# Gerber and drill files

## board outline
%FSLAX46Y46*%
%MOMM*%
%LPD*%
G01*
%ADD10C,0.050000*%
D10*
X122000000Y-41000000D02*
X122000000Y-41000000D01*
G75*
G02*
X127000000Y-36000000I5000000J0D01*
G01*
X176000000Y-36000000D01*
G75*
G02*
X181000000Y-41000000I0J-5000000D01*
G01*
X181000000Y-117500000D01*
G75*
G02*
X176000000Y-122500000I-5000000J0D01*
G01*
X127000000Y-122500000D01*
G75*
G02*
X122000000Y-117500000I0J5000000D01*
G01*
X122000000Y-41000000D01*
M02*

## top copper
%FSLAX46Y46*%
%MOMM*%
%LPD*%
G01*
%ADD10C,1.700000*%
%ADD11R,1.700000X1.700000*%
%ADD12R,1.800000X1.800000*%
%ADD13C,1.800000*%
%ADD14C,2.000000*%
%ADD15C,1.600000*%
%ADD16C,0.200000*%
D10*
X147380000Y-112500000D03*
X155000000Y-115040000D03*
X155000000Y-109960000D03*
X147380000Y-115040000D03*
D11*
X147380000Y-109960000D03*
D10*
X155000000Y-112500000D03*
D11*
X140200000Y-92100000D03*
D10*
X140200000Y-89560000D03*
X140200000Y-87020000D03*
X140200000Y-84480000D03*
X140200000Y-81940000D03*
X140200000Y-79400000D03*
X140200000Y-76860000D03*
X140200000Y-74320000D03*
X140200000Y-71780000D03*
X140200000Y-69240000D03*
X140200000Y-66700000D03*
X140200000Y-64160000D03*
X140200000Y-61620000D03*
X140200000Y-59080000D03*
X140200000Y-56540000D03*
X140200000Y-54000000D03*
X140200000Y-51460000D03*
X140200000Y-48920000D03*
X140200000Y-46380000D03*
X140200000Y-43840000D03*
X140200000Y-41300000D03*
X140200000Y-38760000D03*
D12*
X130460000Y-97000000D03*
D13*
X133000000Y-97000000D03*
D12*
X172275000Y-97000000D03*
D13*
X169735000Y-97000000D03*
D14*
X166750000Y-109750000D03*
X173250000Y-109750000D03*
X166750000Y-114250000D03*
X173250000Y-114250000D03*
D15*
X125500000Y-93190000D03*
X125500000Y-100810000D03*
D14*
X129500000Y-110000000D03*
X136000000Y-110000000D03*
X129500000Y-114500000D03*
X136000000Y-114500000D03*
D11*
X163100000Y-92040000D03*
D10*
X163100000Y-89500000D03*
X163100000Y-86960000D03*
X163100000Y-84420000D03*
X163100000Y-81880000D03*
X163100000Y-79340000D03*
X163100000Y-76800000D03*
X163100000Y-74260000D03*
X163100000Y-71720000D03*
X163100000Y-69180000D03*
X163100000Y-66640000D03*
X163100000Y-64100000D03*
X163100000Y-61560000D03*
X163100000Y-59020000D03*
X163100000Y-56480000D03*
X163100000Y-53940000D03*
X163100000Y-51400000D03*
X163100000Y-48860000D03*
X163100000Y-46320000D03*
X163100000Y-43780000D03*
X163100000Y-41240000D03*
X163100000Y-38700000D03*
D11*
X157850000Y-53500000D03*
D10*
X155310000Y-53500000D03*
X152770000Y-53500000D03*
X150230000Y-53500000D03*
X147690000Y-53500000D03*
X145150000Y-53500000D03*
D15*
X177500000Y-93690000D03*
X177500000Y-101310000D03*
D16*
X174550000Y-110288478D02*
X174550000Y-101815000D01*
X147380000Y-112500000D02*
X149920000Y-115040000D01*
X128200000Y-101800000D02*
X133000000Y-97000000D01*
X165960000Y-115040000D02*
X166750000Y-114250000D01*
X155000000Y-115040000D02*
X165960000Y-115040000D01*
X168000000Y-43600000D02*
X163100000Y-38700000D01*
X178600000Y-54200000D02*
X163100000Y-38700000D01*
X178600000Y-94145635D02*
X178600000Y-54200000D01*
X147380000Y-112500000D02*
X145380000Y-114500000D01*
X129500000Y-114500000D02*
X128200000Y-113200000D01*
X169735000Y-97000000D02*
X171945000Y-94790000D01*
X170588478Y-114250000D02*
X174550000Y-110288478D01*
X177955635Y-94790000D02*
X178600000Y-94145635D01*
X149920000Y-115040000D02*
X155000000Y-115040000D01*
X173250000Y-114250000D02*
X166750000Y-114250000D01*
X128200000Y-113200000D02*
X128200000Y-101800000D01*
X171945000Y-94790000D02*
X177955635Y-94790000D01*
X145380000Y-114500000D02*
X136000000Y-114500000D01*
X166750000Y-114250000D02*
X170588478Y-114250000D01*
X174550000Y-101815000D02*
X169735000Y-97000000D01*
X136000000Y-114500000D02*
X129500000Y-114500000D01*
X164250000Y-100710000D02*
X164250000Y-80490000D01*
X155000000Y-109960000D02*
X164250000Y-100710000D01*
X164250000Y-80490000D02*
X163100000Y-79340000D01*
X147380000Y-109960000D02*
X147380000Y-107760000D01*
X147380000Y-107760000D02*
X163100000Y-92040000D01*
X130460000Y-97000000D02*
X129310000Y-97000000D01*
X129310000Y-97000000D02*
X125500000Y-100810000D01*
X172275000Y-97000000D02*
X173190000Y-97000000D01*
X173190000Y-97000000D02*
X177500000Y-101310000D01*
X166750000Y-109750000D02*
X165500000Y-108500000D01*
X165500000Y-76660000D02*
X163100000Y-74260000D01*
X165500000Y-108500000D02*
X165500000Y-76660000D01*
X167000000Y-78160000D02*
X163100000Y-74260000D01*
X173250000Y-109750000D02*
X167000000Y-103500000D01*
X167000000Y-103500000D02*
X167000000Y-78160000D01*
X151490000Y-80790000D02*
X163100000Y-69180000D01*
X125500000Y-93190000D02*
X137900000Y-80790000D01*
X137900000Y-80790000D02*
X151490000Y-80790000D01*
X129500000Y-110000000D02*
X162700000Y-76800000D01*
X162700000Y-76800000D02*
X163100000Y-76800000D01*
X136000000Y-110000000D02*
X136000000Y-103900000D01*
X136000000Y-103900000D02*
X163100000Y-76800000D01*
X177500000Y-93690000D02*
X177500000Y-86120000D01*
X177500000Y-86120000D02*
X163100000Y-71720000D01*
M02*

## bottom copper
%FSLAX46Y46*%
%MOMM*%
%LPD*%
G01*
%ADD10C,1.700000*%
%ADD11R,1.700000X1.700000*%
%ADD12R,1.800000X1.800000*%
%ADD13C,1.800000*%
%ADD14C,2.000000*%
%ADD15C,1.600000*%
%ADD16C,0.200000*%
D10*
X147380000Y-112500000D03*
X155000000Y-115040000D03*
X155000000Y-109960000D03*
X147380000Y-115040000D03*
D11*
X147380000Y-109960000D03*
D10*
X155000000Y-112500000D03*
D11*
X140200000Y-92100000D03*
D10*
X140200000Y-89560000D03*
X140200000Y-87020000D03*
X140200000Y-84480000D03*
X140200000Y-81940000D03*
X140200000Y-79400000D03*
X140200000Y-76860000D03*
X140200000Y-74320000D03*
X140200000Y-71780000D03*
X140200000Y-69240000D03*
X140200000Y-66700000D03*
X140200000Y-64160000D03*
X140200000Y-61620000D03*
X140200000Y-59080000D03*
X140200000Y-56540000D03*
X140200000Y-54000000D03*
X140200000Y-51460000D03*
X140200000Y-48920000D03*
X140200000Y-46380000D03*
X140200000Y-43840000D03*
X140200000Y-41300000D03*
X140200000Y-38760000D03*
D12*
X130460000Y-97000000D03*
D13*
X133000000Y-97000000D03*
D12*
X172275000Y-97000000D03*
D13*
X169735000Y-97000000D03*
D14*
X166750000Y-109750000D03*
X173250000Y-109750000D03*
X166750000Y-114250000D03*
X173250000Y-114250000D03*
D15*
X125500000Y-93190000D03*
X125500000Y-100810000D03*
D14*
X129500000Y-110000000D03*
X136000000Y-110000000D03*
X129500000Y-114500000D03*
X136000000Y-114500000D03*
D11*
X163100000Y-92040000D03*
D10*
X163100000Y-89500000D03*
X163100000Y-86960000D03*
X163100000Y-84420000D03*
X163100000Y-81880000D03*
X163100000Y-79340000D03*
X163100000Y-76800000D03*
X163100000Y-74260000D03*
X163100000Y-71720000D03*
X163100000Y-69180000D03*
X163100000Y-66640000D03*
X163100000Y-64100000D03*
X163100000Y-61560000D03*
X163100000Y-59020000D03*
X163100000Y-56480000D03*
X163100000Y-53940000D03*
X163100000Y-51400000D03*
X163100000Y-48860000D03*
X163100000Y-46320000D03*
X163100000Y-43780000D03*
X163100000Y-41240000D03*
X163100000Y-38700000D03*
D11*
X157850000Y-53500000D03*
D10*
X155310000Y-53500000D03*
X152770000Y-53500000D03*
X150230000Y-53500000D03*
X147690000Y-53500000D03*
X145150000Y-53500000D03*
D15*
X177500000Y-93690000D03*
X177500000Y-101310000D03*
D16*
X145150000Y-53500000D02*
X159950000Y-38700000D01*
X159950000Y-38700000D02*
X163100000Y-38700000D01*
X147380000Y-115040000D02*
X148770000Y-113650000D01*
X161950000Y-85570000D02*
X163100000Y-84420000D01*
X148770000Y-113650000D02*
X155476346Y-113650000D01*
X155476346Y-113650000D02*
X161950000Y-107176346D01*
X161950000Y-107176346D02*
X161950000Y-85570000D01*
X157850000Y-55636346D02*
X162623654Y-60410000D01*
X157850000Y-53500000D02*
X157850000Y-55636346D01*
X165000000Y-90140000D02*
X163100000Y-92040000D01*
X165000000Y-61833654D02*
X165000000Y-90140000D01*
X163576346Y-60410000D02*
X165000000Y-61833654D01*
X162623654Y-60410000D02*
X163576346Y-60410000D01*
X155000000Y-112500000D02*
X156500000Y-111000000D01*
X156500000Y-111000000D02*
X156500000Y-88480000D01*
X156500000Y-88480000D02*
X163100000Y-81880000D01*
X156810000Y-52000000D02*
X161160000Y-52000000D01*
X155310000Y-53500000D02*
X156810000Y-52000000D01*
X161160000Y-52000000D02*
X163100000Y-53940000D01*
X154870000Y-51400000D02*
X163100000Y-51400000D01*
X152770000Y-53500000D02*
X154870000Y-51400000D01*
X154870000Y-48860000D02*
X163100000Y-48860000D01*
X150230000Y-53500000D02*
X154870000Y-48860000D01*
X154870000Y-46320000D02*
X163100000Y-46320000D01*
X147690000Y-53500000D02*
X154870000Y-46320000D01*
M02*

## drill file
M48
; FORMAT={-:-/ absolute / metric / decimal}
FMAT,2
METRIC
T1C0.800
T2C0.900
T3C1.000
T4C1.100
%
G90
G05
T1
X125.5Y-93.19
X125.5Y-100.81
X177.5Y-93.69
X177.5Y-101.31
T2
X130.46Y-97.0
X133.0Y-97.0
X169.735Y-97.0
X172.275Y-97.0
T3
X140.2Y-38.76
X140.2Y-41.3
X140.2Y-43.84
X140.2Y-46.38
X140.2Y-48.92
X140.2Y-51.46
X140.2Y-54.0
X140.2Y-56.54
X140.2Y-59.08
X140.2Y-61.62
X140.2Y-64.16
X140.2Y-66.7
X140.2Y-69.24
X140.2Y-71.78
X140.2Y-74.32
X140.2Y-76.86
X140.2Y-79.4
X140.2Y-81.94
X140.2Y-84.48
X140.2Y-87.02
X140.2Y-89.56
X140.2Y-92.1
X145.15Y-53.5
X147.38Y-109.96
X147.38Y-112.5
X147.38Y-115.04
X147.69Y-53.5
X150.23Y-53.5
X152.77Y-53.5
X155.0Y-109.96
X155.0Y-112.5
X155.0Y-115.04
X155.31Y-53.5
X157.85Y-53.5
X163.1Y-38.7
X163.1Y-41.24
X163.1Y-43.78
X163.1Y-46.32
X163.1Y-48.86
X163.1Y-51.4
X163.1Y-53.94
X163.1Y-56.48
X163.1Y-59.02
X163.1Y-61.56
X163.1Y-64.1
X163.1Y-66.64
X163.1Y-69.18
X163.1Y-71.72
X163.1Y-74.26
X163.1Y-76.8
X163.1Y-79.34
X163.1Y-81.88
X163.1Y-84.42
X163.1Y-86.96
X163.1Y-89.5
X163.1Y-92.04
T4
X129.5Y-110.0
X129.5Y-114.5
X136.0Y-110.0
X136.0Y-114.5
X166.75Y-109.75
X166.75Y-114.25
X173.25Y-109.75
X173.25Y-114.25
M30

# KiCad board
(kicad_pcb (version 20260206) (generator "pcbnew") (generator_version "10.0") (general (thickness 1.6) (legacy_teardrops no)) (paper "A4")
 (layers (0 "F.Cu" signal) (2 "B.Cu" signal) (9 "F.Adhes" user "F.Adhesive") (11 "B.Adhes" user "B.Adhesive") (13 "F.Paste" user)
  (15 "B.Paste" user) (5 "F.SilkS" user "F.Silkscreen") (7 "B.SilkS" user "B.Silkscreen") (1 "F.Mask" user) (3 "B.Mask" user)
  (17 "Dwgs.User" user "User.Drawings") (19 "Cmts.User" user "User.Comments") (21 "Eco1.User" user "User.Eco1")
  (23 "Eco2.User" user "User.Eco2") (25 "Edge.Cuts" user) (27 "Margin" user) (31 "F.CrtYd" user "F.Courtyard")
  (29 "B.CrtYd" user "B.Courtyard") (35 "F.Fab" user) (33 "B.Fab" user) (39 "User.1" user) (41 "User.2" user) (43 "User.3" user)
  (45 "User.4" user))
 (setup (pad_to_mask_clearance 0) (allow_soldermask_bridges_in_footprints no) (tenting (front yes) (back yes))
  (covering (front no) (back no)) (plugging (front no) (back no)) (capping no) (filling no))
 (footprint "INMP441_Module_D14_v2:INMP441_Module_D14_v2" (layer "F.Cu") (at 151.19 112.5)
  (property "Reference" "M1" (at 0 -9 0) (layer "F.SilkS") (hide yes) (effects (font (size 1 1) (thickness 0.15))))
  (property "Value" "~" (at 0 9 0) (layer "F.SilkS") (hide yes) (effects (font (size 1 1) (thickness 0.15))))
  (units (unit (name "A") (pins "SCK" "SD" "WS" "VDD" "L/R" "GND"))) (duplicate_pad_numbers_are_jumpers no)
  (pad "GND" thru_hole circle (at -3.81 0) (size 1.7 1.7) (drill 1) (layers "*.Cu" "*.Mask" "F.SilkS") (remove_unused_layers no) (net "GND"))
  (pad "L/R" thru_hole circle (at 3.81 2.54) (size 1.7 1.7) (drill 1) (layers "*.Cu" "*.Mask" "F.SilkS") (remove_unused_layers no)
   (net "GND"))
  (pad "SCK" thru_hole circle (at 3.81 -2.54) (size 1.7 1.7) (drill 1) (layers "*.Cu" "*.Mask" "F.SilkS") (remove_unused_layers no)
   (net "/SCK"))
  (pad "SD" thru_hole circle (at -3.81 2.54) (size 1.7 1.7) (drill 1) (layers "*.Cu" "*.Mask" "F.SilkS") (remove_unused_layers no)
   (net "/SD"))
  (pad "VDD" thru_hole rect (at -3.81 -2.54) (size 1.7 1.7) (drill 1) (layers "*.Cu" "*.Mask" "F.SilkS") (remove_unused_layers no)
   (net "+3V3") (thermal_bridge_angle 45))
  (pad "WS" thru_hole circle (at 3.81 0) (size 1.7 1.7) (drill 1) (layers "*.Cu" "*.Mask" "F.SilkS") (remove_unused_layers no) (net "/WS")))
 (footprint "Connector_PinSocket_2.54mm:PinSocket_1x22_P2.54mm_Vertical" (layer "F.Cu") (at 140.2 92.1 180)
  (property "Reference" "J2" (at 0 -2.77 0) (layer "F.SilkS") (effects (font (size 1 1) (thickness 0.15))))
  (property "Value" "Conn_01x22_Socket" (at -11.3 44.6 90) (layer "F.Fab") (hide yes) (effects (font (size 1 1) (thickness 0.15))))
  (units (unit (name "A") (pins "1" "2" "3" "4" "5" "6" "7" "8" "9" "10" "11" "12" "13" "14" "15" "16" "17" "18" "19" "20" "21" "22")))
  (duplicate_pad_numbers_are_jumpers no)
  (pad "1" thru_hole rect (at 0 0 180) (size 1.7 1.7) (drill 1) (layers "*.Cu" "*.Mask") (remove_unused_layers no)
   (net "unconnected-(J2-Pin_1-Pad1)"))
  (pad "2" thru_hole circle (at 0 2.54 180) (size 1.7 1.7) (drill 1) (layers "*.Cu" "*.Mask") (remove_unused_layers no)
   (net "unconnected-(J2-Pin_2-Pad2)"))
  (pad "3" thru_hole circle (at 0 5.08 180) (size 1.7 1.7) (drill 1) (layers "*.Cu" "*.Mask") (remove_unused_layers no)
   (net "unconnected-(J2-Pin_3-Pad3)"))
  (pad "4" thru_hole circle (at 0 7.62 180) (size 1.7 1.7) (drill 1) (layers "*.Cu" "*.Mask") (remove_unused_layers no)
   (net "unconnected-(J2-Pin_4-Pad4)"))
  (pad "5" thru_hole circle (at 0 10.16 180) (size 1.7 1.7) (drill 1) (layers "*.Cu" "*.Mask") (remove_unused_layers no)
   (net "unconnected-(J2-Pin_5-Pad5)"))
  (pad "6" thru_hole circle (at 0 12.7 180) (size 1.7 1.7) (drill 1) (layers "*.Cu" "*.Mask") (remove_unused_layers no)
   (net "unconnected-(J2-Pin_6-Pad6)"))
  (pad "7" thru_hole circle (at 0 15.24 180) (size 1.7 1.7) (drill 1) (layers "*.Cu" "*.Mask") (remove_unused_layers no)
   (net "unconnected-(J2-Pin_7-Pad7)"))
  (pad "8" thru_hole circle (at 0 17.78 180) (size 1.7 1.7) (drill 1) (layers "*.Cu" "*.Mask") (remove_unused_layers no)
   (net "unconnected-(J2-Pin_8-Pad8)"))
  (pad "9" thru_hole circle (at 0 20.32 180) (size 1.7 1.7) (drill 1) (layers "*.Cu" "*.Mask") (remove_unused_layers no)
   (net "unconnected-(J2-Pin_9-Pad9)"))
  (pad "10" thru_hole circle (at 0 22.86 180) (size 1.7 1.7) (drill 1) (layers "*.Cu" "*.Mask") (remove_unused_layers no)
   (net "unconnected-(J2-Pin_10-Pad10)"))
  (pad "11" thru_hole circle (at 0 25.4 180) (size 1.7 1.7) (drill 1) (layers "*.Cu" "*.Mask") (remove_unused_layers no)
   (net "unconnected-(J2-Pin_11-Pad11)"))
  (pad "12" thru_hole circle (at 0 27.94 180) (size 1.7 1.7) (drill 1) (layers "*.Cu" "*.Mask") (remove_unused_layers no)
   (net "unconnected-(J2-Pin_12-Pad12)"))
  (pad "13" thru_hole circle (at 0 30.48 180) (size 1.7 1.7) (drill 1) (layers "*.Cu" "*.Mask") (remove_unused_layers no)
   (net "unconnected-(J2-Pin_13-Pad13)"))
  (pad "14" thru_hole circle (at 0 33.02 180) (size 1.7 1.7) (drill 1) (layers "*.Cu" "*.Mask") (remove_unused_layers no)
   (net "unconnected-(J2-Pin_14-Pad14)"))
  (pad "15" thru_hole circle (at 0 35.56 180) (size 1.7 1.7) (drill 1) (layers "*.Cu" "*.Mask") (remove_unused_layers no)
   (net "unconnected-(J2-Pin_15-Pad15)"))
  (pad "16" thru_hole circle (at 0 38.1 180) (size 1.7 1.7) (drill 1) (layers "*.Cu" "*.Mask") (remove_unused_layers no)
   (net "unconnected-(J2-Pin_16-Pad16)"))
  (pad "17" thru_hole circle (at 0 40.64 180) (size 1.7 1.7) (drill 1) (layers "*.Cu" "*.Mask") (remove_unused_layers no)
   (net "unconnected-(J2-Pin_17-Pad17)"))
  (pad "18" thru_hole circle (at 0 43.18 180) (size 1.7 1.7) (drill 1) (layers "*.Cu" "*.Mask") (remove_unused_layers no)
   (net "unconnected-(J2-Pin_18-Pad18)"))
  (pad "19" thru_hole circle (at 0 45.72 180) (size 1.7 1.7) (drill 1) (layers "*.Cu" "*.Mask") (remove_unused_layers no)
   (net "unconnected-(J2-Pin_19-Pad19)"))
  (pad "20" thru_hole circle (at 0 48.26 180) (size 1.7 1.7) (drill 1) (layers "*.Cu" "*.Mask") (remove_unused_layers no)
   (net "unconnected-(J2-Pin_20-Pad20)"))
  (pad "21" thru_hole circle (at 0 50.8 180) (size 1.7 1.7) (drill 1) (layers "*.Cu" "*.Mask") (remove_unused_layers no)
   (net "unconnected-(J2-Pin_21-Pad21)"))
  (pad "22" thru_hole circle (at 0 53.34 180) (size 1.7 1.7) (drill 1) (layers "*.Cu" "*.Mask") (remove_unused_layers no)
   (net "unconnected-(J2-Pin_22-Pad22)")))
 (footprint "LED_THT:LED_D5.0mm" (layer "F.Cu") (at 130.46 97)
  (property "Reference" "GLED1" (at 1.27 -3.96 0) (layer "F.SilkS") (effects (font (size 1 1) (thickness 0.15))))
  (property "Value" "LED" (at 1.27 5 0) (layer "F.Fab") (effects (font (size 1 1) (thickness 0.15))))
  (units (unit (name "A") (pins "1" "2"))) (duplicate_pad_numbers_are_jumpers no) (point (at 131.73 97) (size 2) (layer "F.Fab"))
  (pad "1" thru_hole rect (at 0 0) (size 1.8 1.8) (drill 0.9) (layers "*.Cu" "*.Mask") (remove_unused_layers no) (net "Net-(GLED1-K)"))
  (pad "2" thru_hole circle (at 2.54 0) (size 1.8 1.8) (drill 0.9) (layers "*.Cu" "*.Mask") (remove_unused_layers no) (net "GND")))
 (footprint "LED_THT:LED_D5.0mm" (layer "F.Cu") (at 172.275 97 180)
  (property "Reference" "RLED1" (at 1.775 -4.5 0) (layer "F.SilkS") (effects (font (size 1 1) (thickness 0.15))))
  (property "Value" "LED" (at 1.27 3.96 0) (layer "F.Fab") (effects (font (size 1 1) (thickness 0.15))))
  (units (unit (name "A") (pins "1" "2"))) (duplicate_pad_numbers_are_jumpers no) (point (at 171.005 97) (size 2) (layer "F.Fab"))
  (pad "1" thru_hole rect (at 0 0 180) (size 1.8 1.8) (drill 0.9) (layers "*.Cu" "*.Mask") (remove_unused_layers no) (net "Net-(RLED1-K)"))
  (pad "2" thru_hole circle (at 2.54 0 180) (size 1.8 1.8) (drill 0.9) (layers "*.Cu" "*.Mask") (remove_unused_layers no) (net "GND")))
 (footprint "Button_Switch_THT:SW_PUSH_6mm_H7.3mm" (layer "F.Cu") (at 166.75 109.75)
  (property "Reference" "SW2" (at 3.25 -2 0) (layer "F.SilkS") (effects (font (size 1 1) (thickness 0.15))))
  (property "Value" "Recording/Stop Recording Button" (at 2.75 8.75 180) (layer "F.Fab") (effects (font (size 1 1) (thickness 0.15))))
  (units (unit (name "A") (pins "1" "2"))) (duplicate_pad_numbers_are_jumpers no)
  (pad "1" thru_hole circle (at 0 0 90) (size 2 2) (drill 1.1) (layers "*.Cu" "*.Mask") (remove_unused_layers no)
   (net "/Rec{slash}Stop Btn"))
  (pad "1" thru_hole circle (at 6.5 0 90) (size 2 2) (drill 1.1) (layers "*.Cu" "*.Mask") (remove_unused_layers no)
   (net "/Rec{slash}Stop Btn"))
  (pad "2" thru_hole circle (at 0 4.5 90) (size 2 2) (drill 1.1) (layers "*.Cu" "*.Mask") (remove_unused_layers no) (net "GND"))
  (pad "2" thru_hole circle (at 6.5 4.5 90) (size 2 2) (drill 1.1) (layers "*.Cu" "*.Mask") (remove_unused_layers no) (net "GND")))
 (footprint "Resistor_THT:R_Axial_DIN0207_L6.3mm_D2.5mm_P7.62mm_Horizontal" (layer "F.Cu") (at 125.5 93.19 -90)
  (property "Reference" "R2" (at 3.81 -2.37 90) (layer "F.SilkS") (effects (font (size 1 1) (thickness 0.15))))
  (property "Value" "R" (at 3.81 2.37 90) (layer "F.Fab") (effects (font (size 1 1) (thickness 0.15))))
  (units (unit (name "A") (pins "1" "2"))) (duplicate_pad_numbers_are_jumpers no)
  (pad "1" thru_hole circle (at 0 0 270) (size 1.6 1.6) (drill 0.8) (layers "*.Cu" "*.Mask") (remove_unused_layers no) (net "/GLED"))
  (pad "2" thru_hole circle (at 7.62 0 270) (size 1.6 1.6) (drill 0.8) (layers "*.Cu" "*.Mask") (remove_unused_layers no)
   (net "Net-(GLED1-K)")))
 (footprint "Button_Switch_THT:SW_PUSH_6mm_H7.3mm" (layer "F.Cu") (at 129.5 110)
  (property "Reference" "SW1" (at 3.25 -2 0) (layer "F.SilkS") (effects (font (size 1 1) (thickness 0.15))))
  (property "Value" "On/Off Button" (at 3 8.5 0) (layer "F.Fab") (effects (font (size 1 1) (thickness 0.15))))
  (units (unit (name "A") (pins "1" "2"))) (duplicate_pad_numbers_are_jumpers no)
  (pad "1" thru_hole circle (at 0 0 90) (size 2 2) (drill 1.1) (layers "*.Cu" "*.Mask") (remove_unused_layers no) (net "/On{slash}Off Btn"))
  (pad "1" thru_hole circle (at 6.5 0 90) (size 2 2) (drill 1.1) (layers "*.Cu" "*.Mask") (remove_unused_layers no)
   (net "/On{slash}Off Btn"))
  (pad "2" thru_hole circle (at 0 4.5 90) (size 2 2) (drill 1.1) (layers "*.Cu" "*.Mask") (remove_unused_layers no) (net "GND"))
  (pad "2" thru_hole circle (at 6.5 4.5 90) (size 2 2) (drill 1.1) (layers "*.Cu" "*.Mask") (remove_unused_layers no) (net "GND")))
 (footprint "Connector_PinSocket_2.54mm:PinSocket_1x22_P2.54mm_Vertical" (layer "F.Cu") (at 163.1 92.04 180)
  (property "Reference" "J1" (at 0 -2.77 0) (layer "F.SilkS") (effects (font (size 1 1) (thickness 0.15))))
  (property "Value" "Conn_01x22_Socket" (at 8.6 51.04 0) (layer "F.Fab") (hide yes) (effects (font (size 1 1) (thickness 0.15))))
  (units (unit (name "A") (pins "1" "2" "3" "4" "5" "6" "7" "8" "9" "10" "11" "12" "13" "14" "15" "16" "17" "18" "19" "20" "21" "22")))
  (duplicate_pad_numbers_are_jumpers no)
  (pad "1" thru_hole rect (at 0 0 180) (size 1.7 1.7) (drill 1) (layers "*.Cu" "*.Mask") (remove_unused_layers no) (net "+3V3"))
  (pad "2" thru_hole circle (at 0 2.54 180) (size 1.7 1.7) (drill 1) (layers "*.Cu" "*.Mask") (remove_unused_layers no)
   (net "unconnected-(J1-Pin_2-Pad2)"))
  (pad "3" thru_hole circle (at 0 5.08 180) (size 1.7 1.7) (drill 1) (layers "*.Cu" "*.Mask") (remove_unused_layers no)
   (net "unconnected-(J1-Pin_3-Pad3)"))
  (pad "4" thru_hole circle (at 0 7.62 180) (size 1.7 1.7) (drill 1) (layers "*.Cu" "*.Mask") (remove_unused_layers no) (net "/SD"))
  (pad "5" thru_hole circle (at 0 10.16 180) (size 1.7 1.7) (drill 1) (layers "*.Cu" "*.Mask") (remove_unused_layers no) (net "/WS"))
  (pad "6" thru_hole circle (at 0 12.7 180) (size 1.7 1.7) (drill 1) (layers "*.Cu" "*.Mask") (remove_unused_layers no) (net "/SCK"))
  (pad "7" thru_hole circle (at 0 15.24 180) (size 1.7 1.7) (drill 1) (layers "*.Cu" "*.Mask") (remove_unused_layers no)
   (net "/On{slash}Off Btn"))
  (pad "8" thru_hole circle (at 0 17.78 180) (size 1.7 1.7) (drill 1) (layers "*.Cu" "*.Mask") (remove_unused_layers no)
   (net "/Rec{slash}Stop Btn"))
  (pad "9" thru_hole circle (at 0 20.32 180) (size 1.7 1.7) (drill 1) (layers "*.Cu" "*.Mask") (remove_unused_layers no) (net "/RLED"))
  (pad "10" thru_hole circle (at 0 22.86 180) (size 1.7 1.7) (drill 1) (layers "*.Cu" "*.Mask") (remove_unused_layers no) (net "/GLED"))
  (pad "11" thru_hole circle (at 0 25.4 180) (size 1.7 1.7) (drill 1) (layers "*.Cu" "*.Mask") (remove_unused_layers no)
   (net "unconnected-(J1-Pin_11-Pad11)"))
  (pad "12" thru_hole circle (at 0 27.94 180) (size 1.7 1.7) (drill 1) (layers "*.Cu" "*.Mask") (remove_unused_layers no)
   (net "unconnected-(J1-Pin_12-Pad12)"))
  (pad "13" thru_hole circle (at 0 30.48 180) (size 1.7 1.7) (drill 1) (layers "*.Cu" "*.Mask") (remove_unused_layers no)
   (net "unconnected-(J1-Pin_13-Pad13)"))
  (pad "14" thru_hole circle (at 0 33.02 180) (size 1.7 1.7) (drill 1) (layers "*.Cu" "*.Mask") (remove_unused_layers no)
   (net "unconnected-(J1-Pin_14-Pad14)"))
  (pad "15" thru_hole circle (at 0 35.56 180) (size 1.7 1.7) (drill 1) (layers "*.Cu" "*.Mask") (remove_unused_layers no)
   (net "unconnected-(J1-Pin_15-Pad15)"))
  (pad "16" thru_hole circle (at 0 38.1 180) (size 1.7 1.7) (drill 1) (layers "*.Cu" "*.Mask") (remove_unused_layers no) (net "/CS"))
  (pad "17" thru_hole circle (at 0 40.64 180) (size 1.7 1.7) (drill 1) (layers "*.Cu" "*.Mask") (remove_unused_layers no) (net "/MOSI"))
  (pad "18" thru_hole circle (at 0 43.18 180) (size 1.7 1.7) (drill 1) (layers "*.Cu" "*.Mask") (remove_unused_layers no) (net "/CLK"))
  (pad "19" thru_hole circle (at 0 45.72 180) (size 1.7 1.7) (drill 1) (layers "*.Cu" "*.Mask") (remove_unused_layers no) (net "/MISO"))
  (pad "20" thru_hole circle (at 0 48.26 180) (size 1.7 1.7) (drill 1) (layers "*.Cu" "*.Mask") (remove_unused_layers no)
   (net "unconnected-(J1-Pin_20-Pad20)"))
  (pad "21" thru_hole circle (at 0 50.8 180) (size 1.7 1.7) (drill 1) (layers "*.Cu" "*.Mask") (remove_unused_layers no)
   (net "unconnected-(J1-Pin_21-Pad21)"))
  (pad "22" thru_hole circle (at 0 53.34 180) (size 1.7 1.7) (drill 1) (layers "*.Cu" "*.Mask") (remove_unused_layers no) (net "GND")))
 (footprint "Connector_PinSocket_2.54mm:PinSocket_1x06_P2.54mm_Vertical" (layer "F.Cu") (at 157.85 53.5 -90)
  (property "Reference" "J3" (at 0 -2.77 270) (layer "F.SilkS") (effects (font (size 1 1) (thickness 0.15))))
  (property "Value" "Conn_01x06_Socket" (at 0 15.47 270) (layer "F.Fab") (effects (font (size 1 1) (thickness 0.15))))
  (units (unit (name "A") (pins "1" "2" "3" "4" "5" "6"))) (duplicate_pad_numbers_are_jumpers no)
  (pad "1" thru_hole rect (at 0 0 270) (size 1.7 1.7) (drill 1) (layers "*.Cu" "*.Mask") (remove_unused_layers no) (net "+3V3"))
  (pad "2" thru_hole circle (at 0 2.54 270) (size 1.7 1.7) (drill 1) (layers "*.Cu" "*.Mask") (remove_unused_layers no) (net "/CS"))
  (pad "3" thru_hole circle (at 0 5.08 270) (size 1.7 1.7) (drill 1) (layers "*.Cu" "*.Mask") (remove_unused_layers no) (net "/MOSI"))
  (pad "4" thru_hole circle (at 0 7.62 270) (size 1.7 1.7) (drill 1) (layers "*.Cu" "*.Mask") (remove_unused_layers no) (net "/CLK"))
  (pad "5" thru_hole circle (at 0 10.16 270) (size 1.7 1.7) (drill 1) (layers "*.Cu" "*.Mask") (remove_unused_layers no) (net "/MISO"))
  (pad "6" thru_hole circle (at 0 12.7 270) (size 1.7 1.7) (drill 1) (layers "*.Cu" "*.Mask") (remove_unused_layers no) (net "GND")))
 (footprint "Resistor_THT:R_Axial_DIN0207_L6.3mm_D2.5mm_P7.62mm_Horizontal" (layer "F.Cu") (at 177.5 93.69 -90)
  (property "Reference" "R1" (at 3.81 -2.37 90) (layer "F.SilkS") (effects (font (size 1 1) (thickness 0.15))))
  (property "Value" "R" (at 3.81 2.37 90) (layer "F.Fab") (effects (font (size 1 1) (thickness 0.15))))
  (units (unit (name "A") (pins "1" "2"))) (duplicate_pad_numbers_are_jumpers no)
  (pad "1" thru_hole circle (at 0 0 270) (size 1.6 1.6) (drill 0.8) (layers "*.Cu" "*.Mask") (remove_unused_layers no) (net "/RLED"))
  (pad "2" thru_hole circle (at 7.62 0 270) (size 1.6 1.6) (drill 0.8) (layers "*.Cu" "*.Mask") (remove_unused_layers no)
   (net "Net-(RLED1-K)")))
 (gr_rect (start 122 36) (end 181 122.5) (radius 5) (stroke (width 0.05) (type solid)) (fill no) (layer "Edge.Cuts"))
 (segment (start 174.55 110.288478) (end 174.55 101.815) (width 0.2) (layer "F.Cu") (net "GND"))
 (segment (start 147.38 112.5) (end 149.92 115.04) (width 0.2) (layer "F.Cu") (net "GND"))
 (segment (start 128.2 101.8) (end 133 97) (width 0.2) (layer "F.Cu") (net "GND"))
 (segment (start 165.96 115.04) (end 166.75 114.25) (width 0.2) (layer "F.Cu") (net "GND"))
 (segment (start 155 115.04) (end 165.96 115.04) (width 0.2) (layer "F.Cu") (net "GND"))
 (segment (start 168 43.6) (end 163.1 38.7) (width 0.2) (layer "F.Cu") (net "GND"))
 (segment (start 178.6 54.2) (end 163.1 38.7) (width 0.2) (layer "F.Cu") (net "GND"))
 (segment (start 178.6 94.145635) (end 178.6 54.2) (width 0.2) (layer "F.Cu") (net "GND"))
 (segment (start 147.38 112.5) (end 145.38 114.5) (width 0.2) (layer "F.Cu") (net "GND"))
 (segment (start 129.5 114.5) (end 128.2 113.2) (width 0.2) (layer "F.Cu") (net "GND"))
 (segment (start 169.735 97) (end 171.945 94.79) (width 0.2) (layer "F.Cu") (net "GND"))
 (segment (start 170.588478 114.25) (end 174.55 110.288478) (width 0.2) (layer "F.Cu") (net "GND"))
 (segment (start 177.955635 94.79) (end 178.6 94.145635) (width 0.2) (layer "F.Cu") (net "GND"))
 (segment (start 149.92 115.04) (end 155 115.04) (width 0.2) (layer "F.Cu") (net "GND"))
 (segment (start 173.25 114.25) (end 166.75 114.25) (width 0.2) (layer "F.Cu") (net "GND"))
 (segment (start 128.2 113.2) (end 128.2 101.8) (width 0.2) (layer "F.Cu") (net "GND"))
 (segment (start 171.945 94.79) (end 177.955635 94.79) (width 0.2) (layer "F.Cu") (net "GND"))
 (segment (start 145.38 114.5) (end 136 114.5) (width 0.2) (layer "F.Cu") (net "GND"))
 (segment (start 166.75 114.25) (end 170.588478 114.25) (width 0.2) (layer "F.Cu") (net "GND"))
 (segment (start 174.55 101.815) (end 169.735 97) (width 0.2) (layer "F.Cu") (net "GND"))
 (segment (start 136 114.5) (end 129.5 114.5) (width 0.2) (layer "F.Cu") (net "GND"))
 (segment (start 145.15 53.5) (end 159.95 38.7) (width 0.2) (layer "B.Cu") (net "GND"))
 (segment (start 159.95 38.7) (end 163.1 38.7) (width 0.2) (layer "B.Cu") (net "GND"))
 (segment (start 164.25 100.71) (end 164.25 80.49) (width 0.2) (layer "F.Cu") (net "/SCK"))
 (segment (start 155 109.96) (end 164.25 100.71) (width 0.2) (layer "F.Cu") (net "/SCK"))
 (segment (start 164.25 80.49) (end 163.1 79.34) (width 0.2) (layer "F.Cu") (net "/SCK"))
 (segment (start 147.38 115.04) (end 148.77 113.65) (width 0.2) (layer "B.Cu") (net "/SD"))
 (segment (start 161.95 85.57) (end 163.1 84.42) (width 0.2) (layer "B.Cu") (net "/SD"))
 (segment (start 148.77 113.65) (end 155.476346 113.65) (width 0.2) (layer "B.Cu") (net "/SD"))
 (segment (start 155.476346 113.65) (end 161.95 107.176346) (width 0.2) (layer "B.Cu") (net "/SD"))
 (segment (start 161.95 107.176346) (end 161.95 85.57) (width 0.2) (layer "B.Cu") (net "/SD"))
 (segment (start 147.38 109.96) (end 147.38 107.76) (width 0.2) (layer "F.Cu") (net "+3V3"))
 (segment (start 147.38 107.76) (end 163.1 92.04) (width 0.2) (layer "F.Cu") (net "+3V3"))
 (segment (start 157.85 55.636346) (end 162.623654 60.41) (width 0.2) (layer "B.Cu") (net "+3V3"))
 (segment (start 157.85 53.5) (end 157.85 55.636346) (width 0.2) (layer "B.Cu") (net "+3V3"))
 (segment (start 165 90.14) (end 163.1 92.04) (width 0.2) (layer "B.Cu") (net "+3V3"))
 (segment (start 165 61.833654) (end 165 90.14) (width 0.2) (layer "B.Cu") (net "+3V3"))
 (segment (start 163.576346 60.41) (end 165 61.833654) (width 0.2) (layer "B.Cu") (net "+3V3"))
 (segment (start 162.623654 60.41) (end 163.576346 60.41) (width 0.2) (layer "B.Cu") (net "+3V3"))
 (segment (start 155 112.5) (end 156.5 111) (width 0.2) (layer "B.Cu") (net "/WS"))
 (segment (start 156.5 111) (end 156.5 88.48) (width 0.2) (layer "B.Cu") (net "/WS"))
 (segment (start 156.5 88.48) (end 163.1 81.88) (width 0.2) (layer "B.Cu") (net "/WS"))
 (segment (start 130.46 97) (end 129.31 97) (width 0.2) (layer "F.Cu") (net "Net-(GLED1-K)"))
 (segment (start 129.31 97) (end 125.5 100.81) (width 0.2) (layer "F.Cu") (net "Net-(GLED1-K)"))
 (segment (start 172.275 97) (end 173.19 97) (width 0.2) (layer "F.Cu") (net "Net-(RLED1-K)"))
 (segment (start 173.19 97) (end 177.5 101.31) (width 0.2) (layer "F.Cu") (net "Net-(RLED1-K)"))
 (segment (start 166.75 109.75) (end 165.5 108.5) (width 0.2) (layer "F.Cu") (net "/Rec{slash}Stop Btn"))
 (segment (start 165.5 76.66) (end 163.1 74.26) (width 0.2) (layer "F.Cu") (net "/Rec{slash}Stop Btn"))
 (segment (start 165.5 108.5) (end 165.5 76.66) (width 0.2) (layer "F.Cu") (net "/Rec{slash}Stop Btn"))
 (segment (start 167 78.16) (end 163.1 74.26) (width 0.2) (layer "F.Cu") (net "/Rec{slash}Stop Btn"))
 (segment (start 173.25 109.75) (end 167 103.5) (width 0.2) (layer "F.Cu") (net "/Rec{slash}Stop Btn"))
 (segment (start 167 103.5) (end 167 78.16) (width 0.2) (layer "F.Cu") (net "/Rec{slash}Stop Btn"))
 (segment (start 151.49 80.79) (end 163.1 69.18) (width 0.2) (layer "F.Cu") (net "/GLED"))
 (segment (start 125.5 93.19) (end 137.9 80.79) (width 0.2) (layer "F.Cu") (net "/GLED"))
 (segment (start 137.9 80.79) (end 151.49 80.79) (width 0.2) (layer "F.Cu") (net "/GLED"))
 (segment (start 129.5 110) (end 162.7 76.8) (width 0.2) (layer "F.Cu") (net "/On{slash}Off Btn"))
 (segment (start 162.7 76.8) (end 163.1 76.8) (width 0.2) (layer "F.Cu") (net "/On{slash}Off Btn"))
 (segment (start 136 110) (end 136 103.9) (width 0.2) (layer "F.Cu") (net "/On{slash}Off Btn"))
 (segment (start 136 103.9) (end 163.1 76.8) (width 0.2) (layer "F.Cu") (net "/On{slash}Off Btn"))
 (segment (start 177.5 93.69) (end 177.5 86.12) (width 0.2) (layer "F.Cu") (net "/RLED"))
 (segment (start 177.5 86.12) (end 163.1 71.72) (width 0.2) (layer "F.Cu") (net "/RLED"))
 (segment (start 156.81 52) (end 161.16 52) (width 0.2) (layer "B.Cu") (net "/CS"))
 (segment (start 155.31 53.5) (end 156.81 52) (width 0.2) (layer "B.Cu") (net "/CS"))
 (segment (start 161.16 52) (end 163.1 53.94) (width 0.2) (layer "B.Cu") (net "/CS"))
 (segment (start 154.87 51.4) (end 163.1 51.4) (width 0.2) (layer "B.Cu") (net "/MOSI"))
 (segment (start 152.77 53.5) (end 154.87 51.4) (width 0.2) (layer "B.Cu") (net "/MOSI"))
 (segment (start 154.87 48.86) (end 163.1 48.86) (width 0.2) (layer "B.Cu") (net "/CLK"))
 (segment (start 150.23 53.5) (end 154.87 48.86) (width 0.2) (layer "B.Cu") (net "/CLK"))
 (segment (start 154.87 46.32) (end 163.1 46.32) (width 0.2) (layer "B.Cu") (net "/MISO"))
 (segment (start 147.69 53.5) (end 154.87 46.32) (width 0.2) (layer "B.Cu") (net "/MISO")))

